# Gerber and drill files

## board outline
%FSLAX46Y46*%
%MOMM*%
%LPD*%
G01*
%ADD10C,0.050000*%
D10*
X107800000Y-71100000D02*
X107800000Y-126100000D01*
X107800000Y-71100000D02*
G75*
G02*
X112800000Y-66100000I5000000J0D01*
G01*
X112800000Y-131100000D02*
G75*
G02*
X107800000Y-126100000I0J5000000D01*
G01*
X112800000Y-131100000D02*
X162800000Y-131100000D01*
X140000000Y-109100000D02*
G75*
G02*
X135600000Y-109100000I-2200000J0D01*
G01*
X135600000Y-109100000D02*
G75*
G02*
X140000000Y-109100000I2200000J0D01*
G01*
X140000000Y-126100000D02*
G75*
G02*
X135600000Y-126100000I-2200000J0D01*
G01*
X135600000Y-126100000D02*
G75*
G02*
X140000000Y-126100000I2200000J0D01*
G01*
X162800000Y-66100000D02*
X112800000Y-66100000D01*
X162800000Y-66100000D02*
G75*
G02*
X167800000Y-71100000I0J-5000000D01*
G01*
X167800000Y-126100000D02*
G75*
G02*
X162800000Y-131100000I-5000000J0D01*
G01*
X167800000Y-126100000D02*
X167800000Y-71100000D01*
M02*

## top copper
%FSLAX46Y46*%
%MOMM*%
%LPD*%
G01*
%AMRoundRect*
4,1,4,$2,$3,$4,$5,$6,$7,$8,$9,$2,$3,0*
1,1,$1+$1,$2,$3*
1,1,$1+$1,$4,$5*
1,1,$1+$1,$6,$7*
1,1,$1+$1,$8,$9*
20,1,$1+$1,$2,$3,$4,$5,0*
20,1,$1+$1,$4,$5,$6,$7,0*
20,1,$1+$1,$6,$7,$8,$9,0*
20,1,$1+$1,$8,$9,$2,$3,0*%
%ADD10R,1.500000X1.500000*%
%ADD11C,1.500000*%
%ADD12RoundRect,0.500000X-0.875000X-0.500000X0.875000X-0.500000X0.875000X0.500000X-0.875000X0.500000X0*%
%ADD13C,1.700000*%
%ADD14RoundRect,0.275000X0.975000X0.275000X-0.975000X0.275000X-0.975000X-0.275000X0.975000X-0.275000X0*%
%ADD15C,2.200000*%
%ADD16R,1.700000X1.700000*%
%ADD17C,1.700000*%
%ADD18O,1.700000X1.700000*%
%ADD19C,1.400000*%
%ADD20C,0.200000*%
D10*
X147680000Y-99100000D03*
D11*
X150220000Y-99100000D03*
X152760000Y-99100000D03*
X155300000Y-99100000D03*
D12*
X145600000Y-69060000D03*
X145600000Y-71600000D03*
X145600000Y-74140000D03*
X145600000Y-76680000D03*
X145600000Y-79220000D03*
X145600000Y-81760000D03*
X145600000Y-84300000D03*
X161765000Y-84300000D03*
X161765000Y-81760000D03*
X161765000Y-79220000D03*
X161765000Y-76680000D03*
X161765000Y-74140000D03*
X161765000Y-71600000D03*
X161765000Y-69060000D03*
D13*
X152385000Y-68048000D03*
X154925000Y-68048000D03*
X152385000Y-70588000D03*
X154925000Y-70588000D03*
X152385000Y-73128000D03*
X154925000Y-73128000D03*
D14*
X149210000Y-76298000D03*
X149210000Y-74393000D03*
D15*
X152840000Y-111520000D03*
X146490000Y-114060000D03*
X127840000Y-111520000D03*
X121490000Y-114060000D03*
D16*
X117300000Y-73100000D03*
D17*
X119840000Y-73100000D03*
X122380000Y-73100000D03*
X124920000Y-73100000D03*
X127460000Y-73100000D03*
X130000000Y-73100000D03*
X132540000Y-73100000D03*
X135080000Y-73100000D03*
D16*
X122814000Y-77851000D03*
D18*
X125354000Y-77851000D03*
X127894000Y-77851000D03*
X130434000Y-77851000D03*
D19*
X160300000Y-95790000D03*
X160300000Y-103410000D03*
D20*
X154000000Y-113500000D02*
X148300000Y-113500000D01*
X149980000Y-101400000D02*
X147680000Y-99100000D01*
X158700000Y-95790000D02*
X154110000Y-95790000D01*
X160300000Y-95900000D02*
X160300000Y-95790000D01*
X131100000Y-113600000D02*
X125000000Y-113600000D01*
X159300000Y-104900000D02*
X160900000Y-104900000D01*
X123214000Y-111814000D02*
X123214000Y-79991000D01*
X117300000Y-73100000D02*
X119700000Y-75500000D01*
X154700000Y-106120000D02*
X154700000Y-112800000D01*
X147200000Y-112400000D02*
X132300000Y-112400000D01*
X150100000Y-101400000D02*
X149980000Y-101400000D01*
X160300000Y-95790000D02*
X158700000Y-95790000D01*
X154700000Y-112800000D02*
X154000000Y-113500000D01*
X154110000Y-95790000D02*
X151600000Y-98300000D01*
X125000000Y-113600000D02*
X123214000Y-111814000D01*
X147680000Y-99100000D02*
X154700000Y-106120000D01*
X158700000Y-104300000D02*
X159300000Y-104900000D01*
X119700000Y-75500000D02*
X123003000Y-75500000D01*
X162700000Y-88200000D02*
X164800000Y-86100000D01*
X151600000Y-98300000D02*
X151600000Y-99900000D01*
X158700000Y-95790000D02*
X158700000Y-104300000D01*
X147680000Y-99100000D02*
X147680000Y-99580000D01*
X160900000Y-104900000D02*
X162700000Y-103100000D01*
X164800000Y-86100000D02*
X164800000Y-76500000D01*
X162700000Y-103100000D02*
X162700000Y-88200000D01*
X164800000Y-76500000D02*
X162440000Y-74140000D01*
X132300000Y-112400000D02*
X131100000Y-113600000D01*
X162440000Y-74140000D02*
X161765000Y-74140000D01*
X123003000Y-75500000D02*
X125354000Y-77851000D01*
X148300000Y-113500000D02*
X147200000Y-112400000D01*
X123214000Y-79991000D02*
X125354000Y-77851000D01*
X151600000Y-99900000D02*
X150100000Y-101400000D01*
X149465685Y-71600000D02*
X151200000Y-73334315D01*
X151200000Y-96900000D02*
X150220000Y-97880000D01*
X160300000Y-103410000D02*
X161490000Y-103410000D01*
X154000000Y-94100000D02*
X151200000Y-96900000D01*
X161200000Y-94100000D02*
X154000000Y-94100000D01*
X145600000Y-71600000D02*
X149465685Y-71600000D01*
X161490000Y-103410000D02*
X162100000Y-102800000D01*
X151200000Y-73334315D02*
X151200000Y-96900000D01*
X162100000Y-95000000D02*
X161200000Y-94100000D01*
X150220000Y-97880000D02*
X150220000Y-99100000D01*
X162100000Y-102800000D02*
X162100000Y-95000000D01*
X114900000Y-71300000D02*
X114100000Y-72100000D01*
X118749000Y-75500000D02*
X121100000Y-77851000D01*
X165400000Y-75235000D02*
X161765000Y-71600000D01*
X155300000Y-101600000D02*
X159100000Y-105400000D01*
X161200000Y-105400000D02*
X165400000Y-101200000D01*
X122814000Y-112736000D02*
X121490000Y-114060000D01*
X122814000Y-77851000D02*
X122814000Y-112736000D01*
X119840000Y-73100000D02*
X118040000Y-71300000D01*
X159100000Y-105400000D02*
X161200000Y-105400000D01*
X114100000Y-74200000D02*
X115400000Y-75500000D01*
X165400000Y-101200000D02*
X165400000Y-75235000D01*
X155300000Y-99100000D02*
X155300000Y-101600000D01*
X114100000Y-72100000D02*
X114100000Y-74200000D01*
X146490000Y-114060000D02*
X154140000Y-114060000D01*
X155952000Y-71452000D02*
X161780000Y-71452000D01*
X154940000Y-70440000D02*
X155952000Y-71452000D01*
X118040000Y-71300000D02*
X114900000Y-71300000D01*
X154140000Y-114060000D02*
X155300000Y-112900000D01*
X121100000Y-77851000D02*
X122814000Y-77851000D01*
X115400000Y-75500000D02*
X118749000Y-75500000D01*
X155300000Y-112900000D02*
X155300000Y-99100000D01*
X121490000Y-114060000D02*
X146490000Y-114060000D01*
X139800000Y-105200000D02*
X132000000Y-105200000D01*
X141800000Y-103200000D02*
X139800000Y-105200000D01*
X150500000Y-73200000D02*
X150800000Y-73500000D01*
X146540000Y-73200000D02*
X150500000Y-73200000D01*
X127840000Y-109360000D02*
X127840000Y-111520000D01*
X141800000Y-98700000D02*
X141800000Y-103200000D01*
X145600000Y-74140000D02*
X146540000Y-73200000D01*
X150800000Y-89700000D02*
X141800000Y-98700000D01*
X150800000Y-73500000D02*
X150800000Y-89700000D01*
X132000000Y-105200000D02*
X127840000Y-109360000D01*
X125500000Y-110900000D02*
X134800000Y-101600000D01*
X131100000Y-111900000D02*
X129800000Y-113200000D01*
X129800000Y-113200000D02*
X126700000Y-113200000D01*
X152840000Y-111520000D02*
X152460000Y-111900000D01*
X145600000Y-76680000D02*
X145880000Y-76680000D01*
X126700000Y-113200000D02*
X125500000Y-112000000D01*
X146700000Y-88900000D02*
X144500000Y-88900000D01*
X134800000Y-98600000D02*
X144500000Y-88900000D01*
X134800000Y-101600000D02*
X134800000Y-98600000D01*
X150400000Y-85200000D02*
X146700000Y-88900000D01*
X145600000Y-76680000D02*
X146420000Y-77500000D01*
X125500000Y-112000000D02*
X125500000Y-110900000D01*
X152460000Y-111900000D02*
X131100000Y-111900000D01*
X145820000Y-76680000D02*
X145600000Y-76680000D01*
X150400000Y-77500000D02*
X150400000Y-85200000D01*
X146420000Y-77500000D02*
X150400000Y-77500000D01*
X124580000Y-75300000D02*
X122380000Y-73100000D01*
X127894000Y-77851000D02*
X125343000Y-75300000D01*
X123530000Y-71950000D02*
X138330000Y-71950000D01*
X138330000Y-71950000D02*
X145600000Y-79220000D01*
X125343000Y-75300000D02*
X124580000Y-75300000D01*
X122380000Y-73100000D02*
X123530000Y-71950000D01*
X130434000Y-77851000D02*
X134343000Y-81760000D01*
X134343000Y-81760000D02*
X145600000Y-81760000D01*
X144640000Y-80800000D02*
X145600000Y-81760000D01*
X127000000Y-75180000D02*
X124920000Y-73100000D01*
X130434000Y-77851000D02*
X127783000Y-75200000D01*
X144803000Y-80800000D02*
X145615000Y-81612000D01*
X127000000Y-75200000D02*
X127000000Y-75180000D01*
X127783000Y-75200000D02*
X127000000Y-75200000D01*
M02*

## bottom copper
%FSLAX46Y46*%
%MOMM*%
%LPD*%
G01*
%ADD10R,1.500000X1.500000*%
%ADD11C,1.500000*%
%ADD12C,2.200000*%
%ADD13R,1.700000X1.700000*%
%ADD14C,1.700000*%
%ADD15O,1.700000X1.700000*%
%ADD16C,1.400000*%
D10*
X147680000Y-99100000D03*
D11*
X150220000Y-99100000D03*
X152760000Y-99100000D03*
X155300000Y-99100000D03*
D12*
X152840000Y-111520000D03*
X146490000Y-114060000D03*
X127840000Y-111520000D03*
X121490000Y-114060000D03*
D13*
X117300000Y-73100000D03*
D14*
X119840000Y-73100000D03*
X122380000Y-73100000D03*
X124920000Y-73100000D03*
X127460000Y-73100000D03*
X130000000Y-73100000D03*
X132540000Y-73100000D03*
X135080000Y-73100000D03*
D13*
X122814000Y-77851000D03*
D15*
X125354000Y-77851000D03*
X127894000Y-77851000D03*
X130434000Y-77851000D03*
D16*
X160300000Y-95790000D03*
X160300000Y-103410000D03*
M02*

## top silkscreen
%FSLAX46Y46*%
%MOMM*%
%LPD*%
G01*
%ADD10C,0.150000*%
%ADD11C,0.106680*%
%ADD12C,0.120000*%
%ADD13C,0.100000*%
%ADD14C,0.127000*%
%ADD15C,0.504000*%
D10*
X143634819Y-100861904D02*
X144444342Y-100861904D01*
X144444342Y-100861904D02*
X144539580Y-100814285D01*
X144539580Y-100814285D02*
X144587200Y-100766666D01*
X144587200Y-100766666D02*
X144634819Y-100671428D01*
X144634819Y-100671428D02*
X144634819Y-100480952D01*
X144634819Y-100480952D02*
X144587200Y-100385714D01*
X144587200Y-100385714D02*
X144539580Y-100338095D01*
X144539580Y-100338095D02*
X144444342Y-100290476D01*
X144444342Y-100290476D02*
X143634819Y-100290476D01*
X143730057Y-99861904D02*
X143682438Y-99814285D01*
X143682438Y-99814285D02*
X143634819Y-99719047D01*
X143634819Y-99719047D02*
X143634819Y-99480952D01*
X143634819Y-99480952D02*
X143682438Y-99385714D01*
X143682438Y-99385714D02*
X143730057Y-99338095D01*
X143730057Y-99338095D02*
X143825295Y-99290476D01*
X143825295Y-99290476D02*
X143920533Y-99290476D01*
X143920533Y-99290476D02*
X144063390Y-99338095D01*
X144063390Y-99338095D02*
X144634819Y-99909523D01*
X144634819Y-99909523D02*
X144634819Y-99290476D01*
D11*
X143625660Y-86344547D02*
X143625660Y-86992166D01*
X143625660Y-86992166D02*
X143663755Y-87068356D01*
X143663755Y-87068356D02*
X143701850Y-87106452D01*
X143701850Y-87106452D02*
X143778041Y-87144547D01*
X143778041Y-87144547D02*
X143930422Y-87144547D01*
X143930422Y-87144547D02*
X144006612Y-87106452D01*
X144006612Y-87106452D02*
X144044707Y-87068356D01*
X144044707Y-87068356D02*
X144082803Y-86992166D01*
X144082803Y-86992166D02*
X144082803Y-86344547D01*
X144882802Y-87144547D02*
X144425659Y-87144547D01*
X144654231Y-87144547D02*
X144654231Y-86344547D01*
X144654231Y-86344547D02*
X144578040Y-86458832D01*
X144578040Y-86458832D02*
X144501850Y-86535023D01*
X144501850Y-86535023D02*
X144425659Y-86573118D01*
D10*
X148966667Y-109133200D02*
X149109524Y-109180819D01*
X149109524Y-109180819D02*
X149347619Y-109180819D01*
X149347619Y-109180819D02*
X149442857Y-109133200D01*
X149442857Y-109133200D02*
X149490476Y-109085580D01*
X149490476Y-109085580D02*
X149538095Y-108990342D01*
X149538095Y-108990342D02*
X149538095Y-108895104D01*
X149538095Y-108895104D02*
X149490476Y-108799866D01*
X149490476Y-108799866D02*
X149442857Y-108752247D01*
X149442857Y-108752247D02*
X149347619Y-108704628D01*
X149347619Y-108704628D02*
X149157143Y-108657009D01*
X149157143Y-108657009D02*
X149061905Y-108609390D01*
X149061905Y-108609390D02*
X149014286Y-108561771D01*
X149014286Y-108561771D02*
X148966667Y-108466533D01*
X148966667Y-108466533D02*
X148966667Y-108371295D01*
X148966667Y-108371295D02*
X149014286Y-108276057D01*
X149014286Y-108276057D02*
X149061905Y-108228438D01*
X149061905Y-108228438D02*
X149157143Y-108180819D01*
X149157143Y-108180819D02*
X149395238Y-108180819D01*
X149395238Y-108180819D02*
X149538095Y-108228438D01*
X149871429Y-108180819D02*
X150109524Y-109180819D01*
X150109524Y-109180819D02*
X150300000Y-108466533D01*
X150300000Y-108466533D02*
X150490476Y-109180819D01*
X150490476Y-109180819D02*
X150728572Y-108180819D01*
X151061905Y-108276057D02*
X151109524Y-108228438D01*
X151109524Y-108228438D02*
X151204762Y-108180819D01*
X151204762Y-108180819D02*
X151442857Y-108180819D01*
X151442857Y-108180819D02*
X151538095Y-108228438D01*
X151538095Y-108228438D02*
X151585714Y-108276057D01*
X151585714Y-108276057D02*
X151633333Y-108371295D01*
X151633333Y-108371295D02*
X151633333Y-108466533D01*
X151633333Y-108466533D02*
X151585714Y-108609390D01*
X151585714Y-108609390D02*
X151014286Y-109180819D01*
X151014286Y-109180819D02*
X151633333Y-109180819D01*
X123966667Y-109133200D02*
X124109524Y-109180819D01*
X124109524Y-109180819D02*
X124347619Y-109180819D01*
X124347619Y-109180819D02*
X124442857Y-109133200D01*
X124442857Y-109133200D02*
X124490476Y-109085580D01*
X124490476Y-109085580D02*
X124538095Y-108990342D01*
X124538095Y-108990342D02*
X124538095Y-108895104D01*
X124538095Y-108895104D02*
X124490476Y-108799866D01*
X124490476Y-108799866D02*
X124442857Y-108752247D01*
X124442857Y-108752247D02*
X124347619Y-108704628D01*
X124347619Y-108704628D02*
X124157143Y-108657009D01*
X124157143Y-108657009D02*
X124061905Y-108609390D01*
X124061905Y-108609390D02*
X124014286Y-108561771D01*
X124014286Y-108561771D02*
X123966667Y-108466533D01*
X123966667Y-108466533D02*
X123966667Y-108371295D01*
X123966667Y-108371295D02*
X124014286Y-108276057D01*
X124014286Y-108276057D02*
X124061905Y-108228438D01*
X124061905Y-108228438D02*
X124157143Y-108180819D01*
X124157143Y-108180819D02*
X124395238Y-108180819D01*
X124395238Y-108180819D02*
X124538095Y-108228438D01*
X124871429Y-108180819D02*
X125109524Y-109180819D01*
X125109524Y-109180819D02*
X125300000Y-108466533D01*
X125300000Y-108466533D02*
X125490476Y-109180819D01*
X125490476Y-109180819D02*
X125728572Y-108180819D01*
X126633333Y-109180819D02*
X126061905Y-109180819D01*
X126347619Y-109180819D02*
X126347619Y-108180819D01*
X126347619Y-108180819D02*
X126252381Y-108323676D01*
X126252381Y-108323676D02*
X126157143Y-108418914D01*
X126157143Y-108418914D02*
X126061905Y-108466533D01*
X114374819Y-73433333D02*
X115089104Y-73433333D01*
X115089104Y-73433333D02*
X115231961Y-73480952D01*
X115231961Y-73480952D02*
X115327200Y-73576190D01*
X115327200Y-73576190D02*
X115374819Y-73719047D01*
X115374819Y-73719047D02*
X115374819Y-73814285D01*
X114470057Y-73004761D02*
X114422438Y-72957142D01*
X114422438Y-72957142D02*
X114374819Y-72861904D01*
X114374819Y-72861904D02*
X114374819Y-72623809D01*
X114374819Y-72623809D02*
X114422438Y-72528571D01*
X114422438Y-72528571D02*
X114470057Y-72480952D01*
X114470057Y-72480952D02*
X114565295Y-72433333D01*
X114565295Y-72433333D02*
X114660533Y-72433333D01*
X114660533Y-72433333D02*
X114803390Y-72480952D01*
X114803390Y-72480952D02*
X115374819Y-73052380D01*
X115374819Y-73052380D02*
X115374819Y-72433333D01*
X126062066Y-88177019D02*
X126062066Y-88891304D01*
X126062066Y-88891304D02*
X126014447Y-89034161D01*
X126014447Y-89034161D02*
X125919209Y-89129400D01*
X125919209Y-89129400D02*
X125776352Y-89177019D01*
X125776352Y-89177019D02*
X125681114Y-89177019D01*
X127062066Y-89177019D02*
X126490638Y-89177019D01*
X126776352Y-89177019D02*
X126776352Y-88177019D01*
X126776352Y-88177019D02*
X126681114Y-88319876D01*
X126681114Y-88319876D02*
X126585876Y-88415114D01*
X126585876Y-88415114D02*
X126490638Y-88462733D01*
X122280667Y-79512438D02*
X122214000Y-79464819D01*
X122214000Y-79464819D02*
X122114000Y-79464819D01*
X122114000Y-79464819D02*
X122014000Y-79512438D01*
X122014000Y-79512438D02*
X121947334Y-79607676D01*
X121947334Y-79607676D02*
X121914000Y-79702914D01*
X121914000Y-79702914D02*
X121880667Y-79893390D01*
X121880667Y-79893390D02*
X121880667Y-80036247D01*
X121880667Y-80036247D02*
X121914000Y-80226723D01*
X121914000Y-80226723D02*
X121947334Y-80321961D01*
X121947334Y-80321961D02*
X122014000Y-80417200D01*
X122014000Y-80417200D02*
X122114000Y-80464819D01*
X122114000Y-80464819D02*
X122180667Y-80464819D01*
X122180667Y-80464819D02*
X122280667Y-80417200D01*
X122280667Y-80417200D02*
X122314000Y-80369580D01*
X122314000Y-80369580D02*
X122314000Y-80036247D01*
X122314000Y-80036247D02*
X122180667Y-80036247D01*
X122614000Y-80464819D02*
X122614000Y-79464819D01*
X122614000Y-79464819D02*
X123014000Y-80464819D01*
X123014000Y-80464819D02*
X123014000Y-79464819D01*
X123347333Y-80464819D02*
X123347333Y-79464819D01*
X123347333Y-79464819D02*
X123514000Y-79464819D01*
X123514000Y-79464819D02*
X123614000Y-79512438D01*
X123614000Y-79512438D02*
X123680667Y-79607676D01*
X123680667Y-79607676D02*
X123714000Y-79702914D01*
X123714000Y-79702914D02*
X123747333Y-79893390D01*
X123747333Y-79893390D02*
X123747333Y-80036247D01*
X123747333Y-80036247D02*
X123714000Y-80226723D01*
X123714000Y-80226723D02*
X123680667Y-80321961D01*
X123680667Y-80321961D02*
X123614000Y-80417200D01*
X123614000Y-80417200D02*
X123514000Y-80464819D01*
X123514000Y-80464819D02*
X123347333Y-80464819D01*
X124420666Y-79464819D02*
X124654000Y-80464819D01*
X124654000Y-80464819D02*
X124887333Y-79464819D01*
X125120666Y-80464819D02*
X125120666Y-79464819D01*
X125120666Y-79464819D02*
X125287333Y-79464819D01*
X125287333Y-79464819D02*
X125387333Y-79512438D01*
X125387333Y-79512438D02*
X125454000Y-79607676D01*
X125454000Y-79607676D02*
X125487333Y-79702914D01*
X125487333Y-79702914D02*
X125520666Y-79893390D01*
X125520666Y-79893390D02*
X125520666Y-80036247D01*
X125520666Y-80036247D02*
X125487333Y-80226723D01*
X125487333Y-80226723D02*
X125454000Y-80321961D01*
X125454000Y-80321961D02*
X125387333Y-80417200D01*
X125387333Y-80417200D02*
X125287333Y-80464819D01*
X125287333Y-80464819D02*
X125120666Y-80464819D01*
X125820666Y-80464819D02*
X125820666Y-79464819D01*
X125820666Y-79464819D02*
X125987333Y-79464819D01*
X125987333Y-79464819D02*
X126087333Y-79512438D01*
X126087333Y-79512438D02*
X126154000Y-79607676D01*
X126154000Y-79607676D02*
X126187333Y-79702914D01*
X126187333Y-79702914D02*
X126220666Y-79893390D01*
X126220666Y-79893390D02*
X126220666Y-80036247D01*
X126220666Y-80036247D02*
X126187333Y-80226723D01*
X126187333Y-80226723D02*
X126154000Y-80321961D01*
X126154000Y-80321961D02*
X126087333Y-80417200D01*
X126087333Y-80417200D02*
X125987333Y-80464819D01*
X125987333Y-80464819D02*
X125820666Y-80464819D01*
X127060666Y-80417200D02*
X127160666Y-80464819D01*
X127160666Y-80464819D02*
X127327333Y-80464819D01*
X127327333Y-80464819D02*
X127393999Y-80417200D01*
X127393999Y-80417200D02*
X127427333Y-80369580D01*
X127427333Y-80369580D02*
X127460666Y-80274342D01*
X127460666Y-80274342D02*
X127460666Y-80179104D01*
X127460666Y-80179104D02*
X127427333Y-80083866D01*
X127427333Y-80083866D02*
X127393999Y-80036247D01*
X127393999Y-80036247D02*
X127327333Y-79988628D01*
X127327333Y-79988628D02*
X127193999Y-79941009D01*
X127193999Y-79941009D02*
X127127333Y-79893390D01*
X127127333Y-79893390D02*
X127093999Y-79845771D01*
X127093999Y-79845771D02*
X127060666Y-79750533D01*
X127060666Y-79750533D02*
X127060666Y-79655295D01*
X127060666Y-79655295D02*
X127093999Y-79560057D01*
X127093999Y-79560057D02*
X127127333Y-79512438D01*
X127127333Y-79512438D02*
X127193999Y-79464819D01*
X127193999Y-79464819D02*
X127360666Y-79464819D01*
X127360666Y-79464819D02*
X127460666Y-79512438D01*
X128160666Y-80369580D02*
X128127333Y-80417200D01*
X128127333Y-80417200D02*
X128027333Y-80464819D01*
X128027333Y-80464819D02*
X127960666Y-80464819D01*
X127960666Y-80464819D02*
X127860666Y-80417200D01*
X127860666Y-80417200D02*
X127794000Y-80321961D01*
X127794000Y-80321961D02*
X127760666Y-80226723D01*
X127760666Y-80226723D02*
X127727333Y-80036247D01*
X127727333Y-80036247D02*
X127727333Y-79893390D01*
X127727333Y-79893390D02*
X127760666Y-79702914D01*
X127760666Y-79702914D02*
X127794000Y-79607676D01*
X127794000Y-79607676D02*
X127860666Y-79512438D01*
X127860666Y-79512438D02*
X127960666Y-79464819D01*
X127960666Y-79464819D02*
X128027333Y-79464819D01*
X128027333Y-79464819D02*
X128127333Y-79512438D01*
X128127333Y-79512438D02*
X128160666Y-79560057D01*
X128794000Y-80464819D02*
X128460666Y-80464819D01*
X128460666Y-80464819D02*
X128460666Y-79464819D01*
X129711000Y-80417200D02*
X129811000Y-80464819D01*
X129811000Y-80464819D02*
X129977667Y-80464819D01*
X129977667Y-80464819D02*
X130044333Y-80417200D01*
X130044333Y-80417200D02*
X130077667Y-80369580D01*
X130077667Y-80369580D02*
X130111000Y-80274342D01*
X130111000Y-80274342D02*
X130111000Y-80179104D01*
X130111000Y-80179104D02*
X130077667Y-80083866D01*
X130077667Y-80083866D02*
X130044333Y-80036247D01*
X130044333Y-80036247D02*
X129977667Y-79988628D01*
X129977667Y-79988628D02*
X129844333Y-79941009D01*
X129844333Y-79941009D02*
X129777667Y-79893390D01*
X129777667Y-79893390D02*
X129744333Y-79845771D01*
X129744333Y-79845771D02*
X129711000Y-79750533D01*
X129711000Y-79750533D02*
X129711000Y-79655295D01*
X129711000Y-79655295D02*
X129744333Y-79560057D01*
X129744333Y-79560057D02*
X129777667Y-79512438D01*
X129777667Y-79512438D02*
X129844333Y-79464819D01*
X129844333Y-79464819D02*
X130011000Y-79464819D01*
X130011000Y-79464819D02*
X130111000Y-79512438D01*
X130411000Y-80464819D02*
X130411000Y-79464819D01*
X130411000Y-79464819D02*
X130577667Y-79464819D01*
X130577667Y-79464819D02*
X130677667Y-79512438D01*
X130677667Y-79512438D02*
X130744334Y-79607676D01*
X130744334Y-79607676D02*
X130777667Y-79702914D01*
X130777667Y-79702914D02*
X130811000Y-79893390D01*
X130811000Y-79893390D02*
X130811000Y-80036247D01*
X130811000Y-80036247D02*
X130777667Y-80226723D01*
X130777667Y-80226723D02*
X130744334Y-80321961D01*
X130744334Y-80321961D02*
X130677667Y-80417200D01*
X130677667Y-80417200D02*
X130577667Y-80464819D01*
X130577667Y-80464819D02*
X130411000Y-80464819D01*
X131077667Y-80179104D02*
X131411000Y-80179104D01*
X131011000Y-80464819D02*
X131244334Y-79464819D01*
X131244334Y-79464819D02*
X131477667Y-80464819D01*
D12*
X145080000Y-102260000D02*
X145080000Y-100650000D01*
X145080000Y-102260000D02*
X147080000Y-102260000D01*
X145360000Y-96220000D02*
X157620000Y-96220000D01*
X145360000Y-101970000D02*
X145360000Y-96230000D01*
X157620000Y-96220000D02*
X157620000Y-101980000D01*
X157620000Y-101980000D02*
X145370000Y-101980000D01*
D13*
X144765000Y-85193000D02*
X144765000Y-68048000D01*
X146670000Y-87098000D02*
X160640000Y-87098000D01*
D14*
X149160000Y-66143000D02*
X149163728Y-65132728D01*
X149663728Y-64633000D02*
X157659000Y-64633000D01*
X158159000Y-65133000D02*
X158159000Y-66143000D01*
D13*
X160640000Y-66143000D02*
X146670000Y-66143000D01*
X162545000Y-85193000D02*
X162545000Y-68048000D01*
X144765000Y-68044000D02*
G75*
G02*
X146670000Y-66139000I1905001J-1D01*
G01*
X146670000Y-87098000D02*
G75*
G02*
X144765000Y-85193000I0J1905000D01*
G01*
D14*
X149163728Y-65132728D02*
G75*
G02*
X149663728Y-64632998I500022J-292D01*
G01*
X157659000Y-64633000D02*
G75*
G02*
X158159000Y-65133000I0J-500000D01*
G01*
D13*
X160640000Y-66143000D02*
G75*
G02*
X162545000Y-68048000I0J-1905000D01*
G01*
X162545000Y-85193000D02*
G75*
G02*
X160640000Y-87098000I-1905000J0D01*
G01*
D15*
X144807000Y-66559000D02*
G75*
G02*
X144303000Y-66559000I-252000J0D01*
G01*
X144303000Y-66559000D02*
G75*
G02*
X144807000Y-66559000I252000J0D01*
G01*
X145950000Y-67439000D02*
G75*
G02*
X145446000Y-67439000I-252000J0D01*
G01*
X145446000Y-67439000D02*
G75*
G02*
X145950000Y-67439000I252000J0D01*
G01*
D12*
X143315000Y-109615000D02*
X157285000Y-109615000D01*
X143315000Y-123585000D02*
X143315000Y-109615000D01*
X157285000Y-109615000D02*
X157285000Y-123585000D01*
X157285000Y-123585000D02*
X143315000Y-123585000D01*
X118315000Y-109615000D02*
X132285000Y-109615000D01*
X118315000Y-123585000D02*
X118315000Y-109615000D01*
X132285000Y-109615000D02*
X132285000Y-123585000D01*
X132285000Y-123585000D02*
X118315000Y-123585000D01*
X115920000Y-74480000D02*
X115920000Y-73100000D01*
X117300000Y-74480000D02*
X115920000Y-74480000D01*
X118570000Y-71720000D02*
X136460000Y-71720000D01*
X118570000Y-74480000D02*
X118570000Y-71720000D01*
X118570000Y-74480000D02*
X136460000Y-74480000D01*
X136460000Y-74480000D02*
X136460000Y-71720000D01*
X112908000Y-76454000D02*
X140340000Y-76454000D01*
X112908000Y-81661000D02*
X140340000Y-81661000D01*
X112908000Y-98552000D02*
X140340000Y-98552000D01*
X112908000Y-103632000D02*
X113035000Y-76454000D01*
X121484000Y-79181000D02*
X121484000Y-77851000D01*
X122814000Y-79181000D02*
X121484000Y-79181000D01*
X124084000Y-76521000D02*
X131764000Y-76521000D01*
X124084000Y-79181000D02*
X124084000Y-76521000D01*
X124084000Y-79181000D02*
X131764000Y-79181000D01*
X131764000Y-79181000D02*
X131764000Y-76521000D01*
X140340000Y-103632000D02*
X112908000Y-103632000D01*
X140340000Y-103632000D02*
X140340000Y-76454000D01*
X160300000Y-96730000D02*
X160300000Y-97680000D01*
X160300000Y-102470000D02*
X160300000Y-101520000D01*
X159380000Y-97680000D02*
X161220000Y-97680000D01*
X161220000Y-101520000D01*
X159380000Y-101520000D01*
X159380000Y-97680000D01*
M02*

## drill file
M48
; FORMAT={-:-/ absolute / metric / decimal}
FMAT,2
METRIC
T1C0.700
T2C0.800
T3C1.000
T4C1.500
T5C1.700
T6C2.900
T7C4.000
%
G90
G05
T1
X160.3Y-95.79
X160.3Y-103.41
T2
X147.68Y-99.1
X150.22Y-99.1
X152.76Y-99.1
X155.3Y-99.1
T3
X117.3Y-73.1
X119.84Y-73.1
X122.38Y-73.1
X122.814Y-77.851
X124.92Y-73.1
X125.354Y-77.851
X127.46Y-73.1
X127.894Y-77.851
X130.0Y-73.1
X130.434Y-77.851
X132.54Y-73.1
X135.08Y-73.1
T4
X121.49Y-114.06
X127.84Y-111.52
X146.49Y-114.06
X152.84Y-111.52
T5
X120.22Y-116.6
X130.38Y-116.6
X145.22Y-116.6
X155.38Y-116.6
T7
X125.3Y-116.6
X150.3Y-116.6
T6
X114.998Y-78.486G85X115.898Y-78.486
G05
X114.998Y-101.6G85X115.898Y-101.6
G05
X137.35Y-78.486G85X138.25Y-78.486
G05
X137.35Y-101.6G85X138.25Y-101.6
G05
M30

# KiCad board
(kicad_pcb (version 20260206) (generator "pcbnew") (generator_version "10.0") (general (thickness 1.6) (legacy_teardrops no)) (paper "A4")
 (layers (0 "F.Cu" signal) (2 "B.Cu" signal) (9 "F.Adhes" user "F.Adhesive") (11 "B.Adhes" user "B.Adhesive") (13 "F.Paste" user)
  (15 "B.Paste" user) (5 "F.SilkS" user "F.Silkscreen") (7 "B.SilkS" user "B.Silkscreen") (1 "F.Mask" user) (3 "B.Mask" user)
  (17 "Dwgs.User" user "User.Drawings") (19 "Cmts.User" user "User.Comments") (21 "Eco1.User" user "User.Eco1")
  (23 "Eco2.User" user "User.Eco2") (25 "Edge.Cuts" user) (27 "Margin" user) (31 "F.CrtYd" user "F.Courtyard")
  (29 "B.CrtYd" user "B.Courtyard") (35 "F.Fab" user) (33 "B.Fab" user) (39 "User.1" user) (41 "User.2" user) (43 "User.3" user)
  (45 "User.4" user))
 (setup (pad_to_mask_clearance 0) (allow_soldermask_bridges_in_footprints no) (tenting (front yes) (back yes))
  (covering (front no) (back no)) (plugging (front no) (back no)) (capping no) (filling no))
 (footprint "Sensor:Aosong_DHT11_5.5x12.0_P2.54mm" (layer "F.Cu") (at 147.68 99.1 90)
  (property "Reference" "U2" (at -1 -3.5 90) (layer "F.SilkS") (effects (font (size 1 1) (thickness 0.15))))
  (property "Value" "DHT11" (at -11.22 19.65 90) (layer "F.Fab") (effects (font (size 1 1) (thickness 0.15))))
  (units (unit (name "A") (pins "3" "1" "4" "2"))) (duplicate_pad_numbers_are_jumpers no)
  (fp_line (start -3.16 -2.6) (end -1.55 -2.6) (stroke (width 0.12) (type solid)) (layer "F.SilkS"))
  (fp_line (start -3.16 -2.6) (end -3.16 -0.6) (stroke (width 0.12) (type solid)) (layer "F.SilkS"))
  (fp_line (start 2.88 -2.32) (end 2.88 9.94) (stroke (width 0.12) (type solid)) (layer "F.SilkS"))
  (fp_line (start -2.87 -2.32) (end 2.87 -2.32) (stroke (width 0.12) (type solid)) (layer "F.SilkS"))
  (fp_line (start 2.88 9.94) (end -2.88 9.94) (stroke (width 0.12) (type solid)) (layer "F.SilkS"))
  (fp_line (start -2.88 9.94) (end -2.88 -2.31) (stroke (width 0.12) (type solid)) (layer "F.SilkS"))
  (pad "1" thru_hole rect (at 0 0 90) (size 1.5 1.5) (drill 0.8) (layers "*.Cu" "*.Mask") (remove_unused_layers no) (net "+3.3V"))
  (pad "2" thru_hole circle (at 0 2.54 90) (size 1.5 1.5) (drill 0.8) (layers "*.Cu" "*.Mask") (remove_unused_layers no) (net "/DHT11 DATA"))
  (pad "3" thru_hole circle (at 0 5.08 90) (size 1.5 1.5) (drill 0.8) (layers "*.Cu" "*.Mask") (remove_unused_layers no)
   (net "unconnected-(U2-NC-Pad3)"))
  (pad "4" thru_hole circle (at 0 7.62 90) (size 1.5 1.5) (drill 0.8) (layers "*.Cu" "*.Mask") (remove_unused_layers no) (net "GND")))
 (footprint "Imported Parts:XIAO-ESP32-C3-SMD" (layer "F.Cu") (at 144.765 87.18)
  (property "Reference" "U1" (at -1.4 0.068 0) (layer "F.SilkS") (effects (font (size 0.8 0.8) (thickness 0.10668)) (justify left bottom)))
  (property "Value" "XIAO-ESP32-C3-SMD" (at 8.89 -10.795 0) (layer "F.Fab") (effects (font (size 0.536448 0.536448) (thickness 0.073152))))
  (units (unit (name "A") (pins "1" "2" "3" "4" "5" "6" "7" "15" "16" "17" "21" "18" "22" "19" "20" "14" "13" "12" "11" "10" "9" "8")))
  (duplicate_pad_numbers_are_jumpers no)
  (fp_line (start 0 -1.987) (end 0 -19.132) (stroke (width 0.1) (type solid)) (layer "F.SilkS"))
  (fp_line (start 1.905 -0.082) (end 15.875 -0.082) (stroke (width 0.1) (type solid)) (layer "F.SilkS"))
  (fp_line (start 4.395 -21.037) (end 4.398728 -22.047272) (stroke (width 0.127) (type solid)) (layer "F.SilkS"))
  (fp_line (start 4.898728 -22.547) (end 12.894 -22.547) (stroke (width 0.127) (type solid)) (layer "F.SilkS"))
  (fp_line (start 13.394 -22.047) (end 13.394 -21.037) (stroke (width 0.127) (type solid)) (layer "F.SilkS"))
  (fp_line (start 15.875 -21.037) (end 1.905 -21.037) (stroke (width 0.1) (type solid)) (layer "F.SilkS"))
  (fp_line (start 17.78 -1.987) (end 17.78 -19.132) (stroke (width 0.1) (type solid)) (layer "F.SilkS"))
  (fp_arc (start 0 -19.136) (mid 0.557962 -20.483038) (end 1.905 -21.041) (stroke (width 0.1) (type solid)) (layer "F.SilkS"))
  (fp_arc (start 1.905 -0.082) (mid 0.557962 -0.639962) (end 0 -1.987) (stroke (width 0.1) (type solid)) (layer "F.SilkS"))
  (fp_arc (start 4.398728 -22.047272) (mid 4.545272 -22.40064) (end 4.898728 -22.547) (stroke (width 0.127) (type default))
   (layer "F.SilkS"))
  (fp_arc (start 12.894 -22.547) (mid 13.247553 -22.400553) (end 13.394 -22.047) (stroke (width 0.127) (type default)) (layer "F.SilkS"))
  (fp_arc (start 15.875 -21.037) (mid 17.222038 -20.479038) (end 17.78 -19.132) (stroke (width 0.1) (type solid)) (layer "F.SilkS"))
  (fp_arc (start 17.78 -1.987) (mid 17.222038 -0.639962) (end 15.875 -0.082) (stroke (width 0.1) (type solid)) (layer "F.SilkS"))
  (fp_circle (center -0.21 -20.621) (end -0.21 -20.875) (stroke (width 0.5) (type solid)) (fill yes) (layer "F.SilkS"))
  (fp_circle (center 0.933 -19.741) (end 0.933 -19.995) (stroke (width 0.5) (type solid)) (fill yes) (layer "F.SilkS"))
  (pad "1" smd roundrect (at 0.835 -18.12) (size 2.75 2) (layers "F.Cu" "F.Mask" "F.Paste") (roundrect_rratio 0.25)
   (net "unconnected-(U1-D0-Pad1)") (solder_mask_margin 0.0508) (thermal_bridge_angle 45))
  (pad "2" smd roundrect (at 0.835 -15.58) (size 2.75 2) (layers "F.Cu" "F.Mask" "F.Paste") (roundrect_rratio 0.25) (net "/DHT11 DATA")
   (solder_mask_margin 0.0508) (thermal_bridge_angle 45))
  (pad "3" smd roundrect (at 0.835 -13.04) (size 2.75 2) (layers "F.Cu" "F.Mask" "F.Paste") (roundrect_rratio 0.25) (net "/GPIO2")
   (solder_mask_margin 0.0508) (thermal_bridge_angle 45))
  (pad "4" smd roundrect (at 0.835 -10.5) (size 2.75 2) (layers "F.Cu" "F.Mask" "F.Paste") (roundrect_rratio 0.25) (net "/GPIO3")
   (solder_mask_margin 0.0508) (thermal_bridge_angle 45))
  (pad "5" smd roundrect (at 0.835 -7.96) (size 2.75 2) (layers "F.Cu" "F.Mask" "F.Paste") (roundrect_rratio 0.25) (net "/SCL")
   (solder_mask_margin 0.0508) (thermal_bridge_angle 45))
  (pad "6" smd roundrect (at 0.835 -5.42) (size 2.75 2) (layers "F.Cu" "F.Mask" "F.Paste") (roundrect_rratio 0.25) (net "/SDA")
   (solder_mask_margin 0.0508) (thermal_bridge_angle 45))
  (pad "7" smd roundrect (at 0.835 -2.88) (size 2.75 2) (layers "F.Cu" "F.Mask" "F.Paste") (roundrect_rratio 0.25)
   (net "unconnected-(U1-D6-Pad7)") (solder_mask_margin 0.0508) (thermal_bridge_angle 45))
  (pad "8" smd roundrect (at 17 -2.88) (size 2.75 2) (layers "F.Cu" "F.Mask" "F.Paste") (roundrect_rratio 0.25)
   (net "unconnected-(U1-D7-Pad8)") (solder_mask_margin 0.0508) (thermal_bridge_angle 45))
  (pad "9" smd roundrect (at 17 -5.42) (size 2.75 2) (layers "F.Cu" "F.Mask" "F.Paste") (roundrect_rratio 0.25)
   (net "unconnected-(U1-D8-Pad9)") (solder_mask_margin 0.0508) (thermal_bridge_angle 45))
  (pad "10" smd roundrect (at 17 -7.96) (size 2.75 2) (layers "F.Cu" "F.Mask" "F.Paste") (roundrect_rratio 0.25)
   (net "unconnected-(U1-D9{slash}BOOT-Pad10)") (solder_mask_margin 0.0508) (thermal_bridge_angle 45))
  (pad "11" smd roundrect (at 17 -10.5) (size 2.75 2) (layers "F.Cu" "F.Mask" "F.Paste") (roundrect_rratio 0.25)
   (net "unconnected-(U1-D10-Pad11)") (solder_mask_margin 0.0508) (thermal_bridge_angle 45))
  (pad "12" smd roundrect (at 17 -13.04) (size 2.75 2) (layers "F.Cu" "F.Mask" "F.Paste") (roundrect_rratio 0.25) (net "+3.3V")
   (solder_mask_margin 0.0508) (thermal_bridge_angle 45))
  (pad "13" smd roundrect (at 17 -15.58) (size 2.75 2) (layers "F.Cu" "F.Mask" "F.Paste") (roundrect_rratio 0.25) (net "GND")
   (solder_mask_margin 0.0508) (thermal_bridge_angle 45))
  (pad "14" smd roundrect (at 17 -18.12) (size 2.75 2) (layers "F.Cu" "F.Mask" "F.Paste") (roundrect_rratio 0.25) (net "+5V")
   (solder_mask_margin 0.0508) (thermal_bridge_angle 45))
  (pad "15" smd circle (at 7.62 -19.132) (size 1.7 1.7) (layers "F.Cu" "F.Mask" "F.Paste") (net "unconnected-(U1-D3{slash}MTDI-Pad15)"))
  (pad "16" smd circle (at 10.16 -19.132) (size 1.7 1.7) (layers "F.Cu" "F.Mask" "F.Paste") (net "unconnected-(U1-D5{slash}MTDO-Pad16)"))
  (pad "17" smd circle (at 7.62 -16.592) (size 1.7 1.7) (layers "F.Cu" "F.Mask" "F.Paste") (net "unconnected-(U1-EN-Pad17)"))
  (pad "18" smd circle (at 10.16 -16.592) (size 1.7 1.7) (layers "F.Cu" "F.Mask" "F.Paste") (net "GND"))
  (pad "19" smd circle (at 7.62 -14.052) (size 1.7 1.7) (layers "F.Cu" "F.Mask" "F.Paste") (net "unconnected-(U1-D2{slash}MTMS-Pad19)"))
  (pad "20" smd circle (at 10.16 -14.052) (size 1.7 1.7) (layers "F.Cu" "F.Mask" "F.Paste") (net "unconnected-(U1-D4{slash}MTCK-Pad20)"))
  (pad "21" smd roundrect (at 4.445 -10.882 180) (size 2.5 1.1) (layers "F.Cu" "F.Mask" "F.Paste") (roundrect_rratio 0.25)
   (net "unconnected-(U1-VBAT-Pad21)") (thermal_bridge_angle 45))
  (pad "22" smd roundrect (at 4.445 -12.787 180) (size 2.5 1.1) (layers "F.Cu" "F.Mask" "F.Paste") (roundrect_rratio 0.25)
   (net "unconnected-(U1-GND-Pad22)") (thermal_bridge_angle 45)))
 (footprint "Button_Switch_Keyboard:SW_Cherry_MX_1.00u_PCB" (layer "F.Cu") (at 152.84 111.52)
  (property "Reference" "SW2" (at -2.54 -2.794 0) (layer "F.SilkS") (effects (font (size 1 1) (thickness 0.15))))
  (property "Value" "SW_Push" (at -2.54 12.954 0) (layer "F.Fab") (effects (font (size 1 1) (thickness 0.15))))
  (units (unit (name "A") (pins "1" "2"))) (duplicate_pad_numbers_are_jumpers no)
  (fp_line (start -9.525 -1.905) (end 4.445 -1.905) (stroke (width 0.12) (type solid)) (layer "F.SilkS"))
  (fp_line (start -9.525 12.065) (end -9.525 -1.905) (stroke (width 0.12) (type solid)) (layer "F.SilkS"))
  (fp_line (start 4.445 -1.905) (end 4.445 12.065) (stroke (width 0.12) (type solid)) (layer "F.SilkS"))
  (fp_line (start 4.445 12.065) (end -9.525 12.065) (stroke (width 0.12) (type solid)) (layer "F.SilkS"))
  (pad "" np_thru_hole circle (at -7.62 5.08) (size 1.7 1.7) (drill 1.7) (layers "*.Cu" "*.Mask"))
  (pad "" np_thru_hole circle (at -2.54 5.08) (size 4 4) (drill 4) (layers "*.Cu" "*.Mask"))
  (pad "" np_thru_hole circle (at 2.54 5.08) (size 1.7 1.7) (drill 1.7) (layers "*.Cu" "*.Mask"))
  (pad "1" thru_hole circle (at 0 0) (size 2.2 2.2) (drill 1.5) (layers "*.Cu" "*.Mask") (remove_unused_layers no) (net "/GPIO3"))
  (pad "2" thru_hole circle (at -6.35 2.54) (size 2.2 2.2) (drill 1.5) (layers "*.Cu" "*.Mask") (remove_unused_layers no) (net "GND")))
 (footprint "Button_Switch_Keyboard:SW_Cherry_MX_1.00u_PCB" (layer "F.Cu") (at 127.84 111.52)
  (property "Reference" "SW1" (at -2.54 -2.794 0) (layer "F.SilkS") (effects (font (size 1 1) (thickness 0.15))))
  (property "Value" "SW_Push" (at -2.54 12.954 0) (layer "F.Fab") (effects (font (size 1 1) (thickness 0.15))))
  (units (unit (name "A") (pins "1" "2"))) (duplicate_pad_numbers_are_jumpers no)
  (fp_line (start -9.525 -1.905) (end 4.445 -1.905) (stroke (width 0.12) (type solid)) (layer "F.SilkS"))
  (fp_line (start -9.525 12.065) (end -9.525 -1.905) (stroke (width 0.12) (type solid)) (layer "F.SilkS"))
  (fp_line (start 4.445 -1.905) (end 4.445 12.065) (stroke (width 0.12) (type solid)) (layer "F.SilkS"))
  (fp_line (start 4.445 12.065) (end -9.525 12.065) (stroke (width 0.12) (type solid)) (layer "F.SilkS"))
  (pad "" np_thru_hole circle (at -7.62 5.08) (size 1.7 1.7) (drill 1.7) (layers "*.Cu" "*.Mask"))
  (pad "" np_thru_hole circle (at -2.54 5.08) (size 4 4) (drill 4) (layers "*.Cu" "*.Mask"))
  (pad "" np_thru_hole circle (at 2.54 5.08) (size 1.7 1.7) (drill 1.7) (layers "*.Cu" "*.Mask"))
  (pad "1" thru_hole circle (at 0 0) (size 2.2 2.2) (drill 1.5) (layers "*.Cu" "*.Mask") (remove_unused_layers no) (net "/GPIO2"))
  (pad "2" thru_hole circle (at -6.35 2.54) (size 2.2 2.2) (drill 1.5) (layers "*.Cu" "*.Mask") (remove_unused_layers no) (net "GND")))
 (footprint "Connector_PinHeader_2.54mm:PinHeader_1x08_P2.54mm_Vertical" (layer "F.Cu") (at 117.3 73.1 90)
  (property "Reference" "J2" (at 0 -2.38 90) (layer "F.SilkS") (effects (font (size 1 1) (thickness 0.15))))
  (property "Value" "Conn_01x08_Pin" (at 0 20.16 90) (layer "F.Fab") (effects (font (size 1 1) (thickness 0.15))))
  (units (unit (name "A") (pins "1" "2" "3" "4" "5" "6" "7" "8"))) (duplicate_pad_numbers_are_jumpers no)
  (fp_line (start -1.38 -1.38) (end 0 -1.38) (stroke (width 0.12) (type solid)) (layer "F.SilkS"))
  (fp_line (start -1.38 0) (end -1.38 -1.38) (stroke (width 0.12) (type solid)) (layer "F.SilkS"))
  (fp_line (start 1.38 1.27) (end 1.38 19.16) (stroke (width 0.12) (type solid)) (layer "F.SilkS"))
  (fp_line (start -1.38 1.27) (end 1.38 1.27) (stroke (width 0.12) (type solid)) (layer "F.SilkS"))
  (fp_line (start -1.38 1.27) (end -1.38 19.16) (stroke (width 0.12) (type solid)) (layer "F.SilkS"))
  (fp_line (start -1.38 19.16) (end 1.38 19.16) (stroke (width 0.12) (type solid)) (layer "F.SilkS"))
  (pad "1" thru_hole rect (at 0 0 90) (size 1.7 1.7) (drill 1) (layers "*.Cu" "*.Mask") (remove_unused_layers no) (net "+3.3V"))
  (pad "2" thru_hole circle (at 0 2.54 90) (size 1.7 1.7) (drill 1) (layers "*.Cu" "*.Mask") (remove_unused_layers no) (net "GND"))
  (pad "3" thru_hole circle (at 0 5.08 90) (size 1.7 1.7) (drill 1) (layers "*.Cu" "*.Mask") (remove_unused_layers no) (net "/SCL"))
  (pad "4" thru_hole circle (at 0 7.62 90) (size 1.7 1.7) (drill 1) (layers "*.Cu" "*.Mask") (remove_unused_layers no) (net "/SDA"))
  (pad "5" thru_hole circle (at 0 10.16 90) (size 1.7 1.7) (drill 1) (layers "*.Cu" "*.Mask") (remove_unused_layers no)
   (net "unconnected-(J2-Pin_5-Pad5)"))
  (pad "6" thru_hole circle (at 0 12.7 90) (size 1.7 1.7) (drill 1) (layers "*.Cu" "*.Mask") (remove_unused_layers no)
   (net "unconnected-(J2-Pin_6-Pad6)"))
  (pad "7" thru_hole circle (at 0 15.24 90) (size 1.7 1.7) (drill 1) (layers "*.Cu" "*.Mask") (remove_unused_layers no)
   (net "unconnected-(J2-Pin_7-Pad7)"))
  (pad "8" thru_hole circle (at 0 17.78 90) (size 1.7 1.7) (drill 1) (layers "*.Cu" "*.Mask") (remove_unused_layers no)
   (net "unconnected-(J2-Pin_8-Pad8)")))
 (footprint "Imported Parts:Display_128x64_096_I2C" (layer "F.Cu") (at 126.624 77.851)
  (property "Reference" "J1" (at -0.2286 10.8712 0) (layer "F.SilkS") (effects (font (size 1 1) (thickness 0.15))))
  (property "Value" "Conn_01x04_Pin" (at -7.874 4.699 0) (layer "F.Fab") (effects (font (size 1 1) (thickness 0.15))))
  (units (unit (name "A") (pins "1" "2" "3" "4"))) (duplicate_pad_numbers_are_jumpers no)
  (fp_line (start -13.716 -1.397) (end 13.716 -1.397) (stroke (width 0.12) (type solid)) (layer "F.SilkS"))
  (fp_line (start -13.716 3.81) (end 13.716 3.81) (stroke (width 0.12) (type solid)) (layer "F.SilkS"))
  (fp_line (start -13.716 20.701) (end 13.716 20.701) (stroke (width 0.12) (type solid)) (layer "F.SilkS"))
  (fp_line (start -13.716 25.781) (end -13.589 -1.397) (stroke (width 0.12) (type solid)) (layer "F.SilkS"))
  (fp_line (start -5.14 1.33) (end -5.14 0) (stroke (width 0.12) (type solid)) (layer "F.SilkS"))
  (fp_line (start -3.81 1.33) (end -5.14 1.33) (stroke (width 0.12) (type solid)) (layer "F.SilkS"))
  (fp_line (start -2.54 -1.33) (end 5.14 -1.33) (stroke (width 0.12) (type solid)) (layer "F.SilkS"))
  (fp_line (start -2.54 1.33) (end -2.54 -1.33) (stroke (width 0.12) (type solid)) (layer "F.SilkS"))
  (fp_line (start -2.54 1.33) (end 5.14 1.33) (stroke (width 0.12) (type solid)) (layer "F.SilkS"))
  (fp_line (start 5.14 1.33) (end 5.14 -1.33) (stroke (width 0.12) (type solid)) (layer "F.SilkS"))
  (fp_line (start 13.716 25.781) (end -13.716 25.781) (stroke (width 0.12) (type solid)) (layer "F.SilkS"))
  (fp_line (start 13.716 25.781) (end 13.716 -1.397) (stroke (width 0.12) (type solid)) (layer "F.SilkS"))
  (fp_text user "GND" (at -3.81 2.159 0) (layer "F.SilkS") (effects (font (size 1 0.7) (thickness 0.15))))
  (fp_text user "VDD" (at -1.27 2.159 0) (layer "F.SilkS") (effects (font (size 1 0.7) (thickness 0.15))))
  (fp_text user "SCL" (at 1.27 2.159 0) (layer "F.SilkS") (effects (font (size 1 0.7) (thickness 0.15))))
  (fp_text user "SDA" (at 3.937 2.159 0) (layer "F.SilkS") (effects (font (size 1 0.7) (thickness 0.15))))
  (pad "" np_thru_hole oval (at -11.176 0.635) (size 3.8 2.9) (drill oval 3.8 2.9) (layers "*.Cu" "*.Mask"))
  (pad "" np_thru_hole oval (at -11.176 23.749) (size 3.8 2.9) (drill oval 3.8 2.9) (layers "*.Cu" "*.Mask"))
  (pad "" np_thru_hole oval (at 11.176 0.635) (size 3.8 2.9) (drill oval 3.8 2.9) (layers "*.Cu" "*.Mask"))
  (pad "" np_thru_hole oval (at 11.176 23.749) (size 3.8 2.9) (drill oval 3.8 2.9) (layers "*.Cu" "*.Mask"))
  (pad "1" thru_hole rect (at -3.81 0 90) (size 1.7 1.7) (drill 1) (layers "*.Cu" "*.Mask") (remove_unused_layers no) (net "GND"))
  (pad "2" thru_hole oval (at -1.27 0 90) (size 1.7 1.7) (drill 1) (layers "*.Cu" "*.Mask") (remove_unused_layers no) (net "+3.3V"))
  (pad "3" thru_hole oval (at 1.27 0 90) (size 1.7 1.7) (drill 1) (layers "*.Cu" "*.Mask") (remove_unused_layers no) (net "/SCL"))
  (pad "4" thru_hole oval (at 3.81 0 90) (size 1.7 1.7) (drill 1) (layers "*.Cu" "*.Mask") (remove_unused_layers no) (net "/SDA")))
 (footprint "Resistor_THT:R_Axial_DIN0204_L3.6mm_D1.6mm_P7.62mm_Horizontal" (layer "F.Cu") (at 160.3 95.79 -90)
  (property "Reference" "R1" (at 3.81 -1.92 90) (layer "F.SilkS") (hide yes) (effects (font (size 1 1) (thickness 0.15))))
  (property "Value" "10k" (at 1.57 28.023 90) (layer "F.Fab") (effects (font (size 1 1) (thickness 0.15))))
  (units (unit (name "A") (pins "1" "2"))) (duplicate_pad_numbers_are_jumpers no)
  (fp_line (start 0.94 0) (end 1.89 0) (stroke (width 0.12) (type solid)) (layer "F.SilkS"))
  (fp_line (start 6.68 0) (end 5.73 0) (stroke (width 0.12) (type solid)) (layer "F.SilkS"))
  (fp_rect (start 1.89 -0.92) (end 5.73 0.92) (stroke (width 0.12) (type solid)) (fill no) (layer "F.SilkS"))
  (pad "1" thru_hole circle (at 0 0 270) (size 1.4 1.4) (drill 0.7) (layers "*.Cu" "*.Mask") (remove_unused_layers no) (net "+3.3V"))
  (pad "2" thru_hole circle (at 7.62 0 270) (size 1.4 1.4) (drill 0.7) (layers "*.Cu" "*.Mask") (remove_unused_layers no)
   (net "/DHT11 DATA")))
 (gr_line (start 107.8 71.1) (end 107.8 126.1) (stroke (width 0.05) (type default)) (layer "Edge.Cuts"))
 (gr_arc (start 107.8 71.1) (mid 109.264466 67.564466) (end 112.8 66.1) (stroke (width 0.05) (type default)) (layer "Edge.Cuts"))
 (gr_arc (start 112.8 131.1) (mid 109.264466 129.635534) (end 107.8 126.1) (stroke (width 0.05) (type default)) (layer "Edge.Cuts"))
 (gr_line (start 112.8 131.1) (end 162.8 131.1) (stroke (width 0.05) (type default)) (layer "Edge.Cuts"))
 (gr_circle (center 137.8 109.1) (end 140 109.1) (stroke (width 0.05) (type default)) (fill no) (layer "Edge.Cuts"))
 (gr_circle (center 137.8 126.1) (end 140 126.1) (stroke (width 0.05) (type default)) (fill no) (layer "Edge.Cuts"))
 (gr_line (start 162.8 66.1) (end 112.8 66.1) (stroke (width 0.05) (type default)) (layer "Edge.Cuts"))
 (gr_arc (start 162.8 66.1) (mid 166.335534 67.564466) (end 167.8 71.1) (stroke (width 0.05) (type default)) (layer "Edge.Cuts"))
 (gr_arc (start 167.8 126.1) (mid 166.335534 129.635534) (end 162.8 131.1) (stroke (width 0.05) (type default)) (layer "Edge.Cuts"))
 (gr_line (start 167.8 126.1) (end 167.8 71.1) (stroke (width 0.05) (type default)) (layer "Edge.Cuts"))
 (segment (start 154 113.5) (end 148.3 113.5) (width 0.2) (layer "F.Cu") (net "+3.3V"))
 (segment (start 149.98 101.4) (end 147.68 99.1) (width 0.2) (layer "F.Cu") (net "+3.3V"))
 (segment (start 158.7 95.79) (end 154.11 95.79) (width 0.2) (layer "F.Cu") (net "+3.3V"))
 (segment (start 160.3 95.9) (end 160.3 95.79) (width 0.2) (layer "F.Cu") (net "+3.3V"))
 (segment (start 131.1 113.6) (end 125 113.6) (width 0.2) (layer "F.Cu") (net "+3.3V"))
 (segment (start 159.3 104.9) (end 160.9 104.9) (width 0.2) (layer "F.Cu") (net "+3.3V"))
 (segment (start 123.214 111.814) (end 123.214 79.991) (width 0.2) (layer "F.Cu") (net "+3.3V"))
 (segment (start 117.3 73.1) (end 119.7 75.5) (width 0.2) (layer "F.Cu") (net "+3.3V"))
 (segment (start 154.7 106.12) (end 154.7 112.8) (width 0.2) (layer "F.Cu") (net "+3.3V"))
 (segment (start 147.2 112.4) (end 132.3 112.4) (width 0.2) (layer "F.Cu") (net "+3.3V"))
 (segment (start 150.1 101.4) (end 149.98 101.4) (width 0.2) (layer "F.Cu") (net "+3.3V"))
 (segment (start 160.3 95.79) (end 158.7 95.79) (width 0.2) (layer "F.Cu") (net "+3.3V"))
 (segment (start 154.7 112.8) (end 154 113.5) (width 0.2) (layer "F.Cu") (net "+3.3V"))
 (segment (start 154.11 95.79) (end 151.6 98.3) (width 0.2) (layer "F.Cu") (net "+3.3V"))
 (segment (start 125 113.6) (end 123.214 111.814) (width 0.2) (layer "F.Cu") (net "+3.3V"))
 (segment (start 147.68 99.1) (end 154.7 106.12) (width 0.2) (layer "F.Cu") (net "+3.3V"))
 (segment (start 158.7 104.3) (end 159.3 104.9) (width 0.2) (layer "F.Cu") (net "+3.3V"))
 (segment (start 119.7 75.5) (end 123.003 75.5) (width 0.2) (layer "F.Cu") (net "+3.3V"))
 (segment (start 162.7 88.2) (end 164.8 86.1) (width 0.2) (layer "F.Cu") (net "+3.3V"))
 (segment (start 151.6 98.3) (end 151.6 99.9) (width 0.2) (layer "F.Cu") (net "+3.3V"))
 (segment (start 158.7 95.79) (end 158.7 104.3) (width 0.2) (layer "F.Cu") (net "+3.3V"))
 (segment (start 147.68 99.1) (end 147.68 99.58) (width 0.2) (layer "F.Cu") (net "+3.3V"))
 (segment (start 160.9 104.9) (end 162.7 103.1) (width 0.2) (layer "F.Cu") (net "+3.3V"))
 (segment (start 164.8 86.1) (end 164.8 76.5) (width 0.2) (layer "F.Cu") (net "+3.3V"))
 (segment (start 162.7 103.1) (end 162.7 88.2) (width 0.2) (layer "F.Cu") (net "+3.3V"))
 (segment (start 164.8 76.5) (end 162.44 74.14) (width 0.2) (layer "F.Cu") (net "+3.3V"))
 (segment (start 132.3 112.4) (end 131.1 113.6) (width 0.2) (layer "F.Cu") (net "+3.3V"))
 (segment (start 162.44 74.14) (end 161.765 74.14) (width 0.2) (layer "F.Cu") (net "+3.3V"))
 (segment (start 123.003 75.5) (end 125.354 77.851) (width 0.2) (layer "F.Cu") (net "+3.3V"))
 (segment (start 148.3 113.5) (end 147.2 112.4) (width 0.2) (layer "F.Cu") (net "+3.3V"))
 (segment (start 123.214 79.991) (end 125.354 77.851) (width 0.2) (layer "F.Cu") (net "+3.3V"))
 (segment (start 151.6 99.9) (end 150.1 101.4) (width 0.2) (layer "F.Cu") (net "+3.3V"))
 (segment (start 149.465685 71.6) (end 151.2 73.334315) (width 0.2) (layer "F.Cu") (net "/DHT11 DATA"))
 (segment (start 151.2 96.9) (end 150.22 97.88) (width 0.2) (layer "F.Cu") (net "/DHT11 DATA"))
 (segment (start 160.3 103.41) (end 161.49 103.41) (width 0.2) (layer "F.Cu") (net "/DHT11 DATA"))
 (segment (start 154 94.1) (end 151.2 96.9) (width 0.2) (layer "F.Cu") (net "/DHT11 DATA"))
 (segment (start 161.2 94.1) (end 154 94.1) (width 0.2) (layer "F.Cu") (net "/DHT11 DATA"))
 (segment (start 145.6 71.6) (end 149.465685 71.6) (width 0.2) (layer "F.Cu") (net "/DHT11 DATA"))
 (segment (start 161.49 103.41) (end 162.1 102.8) (width 0.2) (layer "F.Cu") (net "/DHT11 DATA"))
 (segment (start 151.2 73.334315) (end 151.2 96.9) (width 0.2) (layer "F.Cu") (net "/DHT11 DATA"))
 (segment (start 162.1 95) (end 161.2 94.1) (width 0.2) (layer "F.Cu") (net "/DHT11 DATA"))
 (segment (start 150.22 97.88) (end 150.22 99.1) (width 0.2) (layer "F.Cu") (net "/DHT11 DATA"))
 (segment (start 162.1 102.8) (end 162.1 95) (width 0.2) (layer "F.Cu") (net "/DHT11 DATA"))
 (segment (start 114.9 71.3) (end 114.1 72.1) (width 0.2) (layer "F.Cu") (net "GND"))
 (segment (start 118.749 75.5) (end 121.1 77.851) (width 0.2) (layer "F.Cu") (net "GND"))
 (segment (start 165.4 75.235) (end 161.765 71.6) (width 0.2) (layer "F.Cu") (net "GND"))
 (segment (start 155.3 101.6) (end 159.1 105.4) (width 0.2) (layer "F.Cu") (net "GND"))
 (segment (start 161.2 105.4) (end 165.4 101.2) (width 0.2) (layer "F.Cu") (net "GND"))
 (segment (start 122.814 112.736) (end 121.49 114.06) (width 0.2) (layer "F.Cu") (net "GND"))
 (segment (start 122.814 77.851) (end 122.814 112.736) (width 0.2) (layer "F.Cu") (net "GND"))
 (segment (start 119.84 73.1) (end 118.04 71.3) (width 0.2) (layer "F.Cu") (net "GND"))
 (segment (start 159.1 105.4) (end 161.2 105.4) (width 0.2) (layer "F.Cu") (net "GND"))
 (segment (start 114.1 74.2) (end 115.4 75.5) (width 0.2) (layer "F.Cu") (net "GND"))
 (segment (start 165.4 101.2) (end 165.4 75.235) (width 0.2) (layer "F.Cu") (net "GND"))
 (segment (start 155.3 99.1) (end 155.3 101.6) (width 0.2) (layer "F.Cu") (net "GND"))
 (segment (start 114.1 72.1) (end 114.1 74.2) (width 0.2) (layer "F.Cu") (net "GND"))
 (segment (start 146.49 114.06) (end 154.14 114.06) (width 0.2) (layer "F.Cu") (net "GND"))
 (segment (start 155.952 71.452) (end 161.78 71.452) (width 0.2) (layer "F.Cu") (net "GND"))
 (segment (start 154.94 70.44) (end 155.952 71.452) (width 0.2) (layer "F.Cu") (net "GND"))
 (segment (start 118.04 71.3) (end 114.9 71.3) (width 0.2) (layer "F.Cu") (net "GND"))
 (segment (start 154.14 114.06) (end 155.3 112.9) (width 0.2) (layer "F.Cu") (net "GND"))
 (segment (start 121.1 77.851) (end 122.814 77.851) (width 0.2) (layer "F.Cu") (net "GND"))
 (segment (start 115.4 75.5) (end 118.749 75.5) (width 0.2) (layer "F.Cu") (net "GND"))
 (segment (start 155.3 112.9) (end 155.3 99.1) (width 0.2) (layer "F.Cu") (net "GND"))
 (segment (start 121.49 114.06) (end 146.49 114.06) (width 0.2) (layer "F.Cu") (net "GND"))
 (segment (start 139.8 105.2) (end 132 105.2) (width 0.2) (layer "F.Cu") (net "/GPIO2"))
 (segment (start 141.8 103.2) (end 139.8 105.2) (width 0.2) (layer "F.Cu") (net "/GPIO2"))
 (segment (start 150.5 73.2) (end 150.8 73.5) (width 0.2) (layer "F.Cu") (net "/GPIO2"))
 (segment (start 146.54 73.2) (end 150.5 73.2) (width 0.2) (layer "F.Cu") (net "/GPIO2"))
 (segment (start 127.84 109.36) (end 127.84 111.52) (width 0.2) (layer "F.Cu") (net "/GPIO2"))
 (segment (start 141.8 98.7) (end 141.8 103.2) (width 0.2) (layer "F.Cu") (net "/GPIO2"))
 (segment (start 145.6 74.14) (end 146.54 73.2) (width 0.2) (layer "F.Cu") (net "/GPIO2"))
 (segment (start 150.8 89.7) (end 141.8 98.7) (width 0.2) (layer "F.Cu") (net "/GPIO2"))
 (segment (start 150.8 73.5) (end 150.8 89.7) (width 0.2) (layer "F.Cu") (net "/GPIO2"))
 (segment (start 132 105.2) (end 127.84 109.36) (width 0.2) (layer "F.Cu") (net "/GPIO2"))
 (segment (start 125.5 110.9) (end 134.8 101.6) (width 0.2) (layer "F.Cu") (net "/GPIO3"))
 (segment (start 131.1 111.9) (end 129.8 113.2) (width 0.2) (layer "F.Cu") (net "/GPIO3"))
 (segment (start 129.8 113.2) (end 126.7 113.2) (width 0.2) (layer "F.Cu") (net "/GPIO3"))
 (segment (start 152.84 111.52) (end 152.46 111.9) (width 0.2) (layer "F.Cu") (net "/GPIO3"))
 (segment (start 145.6 76.68) (end 145.88 76.68) (width 0.2) (layer "F.Cu") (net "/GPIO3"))
 (segment (start 126.7 113.2) (end 125.5 112) (width 0.2) (layer "F.Cu") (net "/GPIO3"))
 (segment (start 146.7 88.9) (end 144.5 88.9) (width 0.2) (layer "F.Cu") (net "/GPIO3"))
 (segment (start 134.8 98.6) (end 144.5 88.9) (width 0.2) (layer "F.Cu") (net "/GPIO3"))
 (segment (start 134.8 101.6) (end 134.8 98.6) (width 0.2) (layer "F.Cu") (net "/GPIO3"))
 (segment (start 150.4 85.2) (end 146.7 88.9) (width 0.2) (layer "F.Cu") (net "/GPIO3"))
 (segment (start 145.6 76.68) (end 146.42 77.5) (width 0.2) (layer "F.Cu") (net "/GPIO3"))
 (segment (start 125.5 112) (end 125.5 110.9) (width 0.2) (layer "F.Cu") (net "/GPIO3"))
 (segment (start 152.46 111.9) (end 131.1 111.9) (width 0.2) (layer "F.Cu") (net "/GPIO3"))
 (segment (start 145.82 76.68) (end 145.6 76.68) (width 0.2) (layer "F.Cu") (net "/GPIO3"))
 (segment (start 150.4 77.5) (end 150.4 85.2) (width 0.2) (layer "F.Cu") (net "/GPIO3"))
 (segment (start 146.42 77.5) (end 150.4 77.5) (width 0.2) (layer "F.Cu") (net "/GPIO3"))
 (segment (start 124.58 75.3) (end 122.38 73.1) (width 0.2) (layer "F.Cu") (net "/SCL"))
 (segment (start 127.894 77.851) (end 125.343 75.3) (width 0.2) (layer "F.Cu") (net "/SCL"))
 (segment (start 123.53 71.95) (end 138.33 71.95) (width 0.2) (layer "F.Cu") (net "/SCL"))
 (segment (start 138.33 71.95) (end 145.6 79.22) (width 0.2) (layer "F.Cu") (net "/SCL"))
 (segment (start 125.343 75.3) (end 124.58 75.3) (width 0.2) (layer "F.Cu") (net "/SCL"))
 (segment (start 122.38 73.1) (end 123.53 71.95) (width 0.2) (layer "F.Cu") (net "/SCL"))
 (segment (start 130.434 77.851) (end 134.343 81.76) (width 0.2) (layer "F.Cu") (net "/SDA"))
 (segment (start 134.343 81.76) (end 145.6 81.76) (width 0.2) (layer "F.Cu") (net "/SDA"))
 (segment (start 144.64 80.8) (end 145.6 81.76) (width 0.2) (layer "F.Cu") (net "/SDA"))
 (segment (start 127 75.18) (end 124.92 73.1) (width 0.2) (layer "F.Cu") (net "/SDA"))
 (segment (start 130.434 77.851) (end 127.783 75.2) (width 0.2) (layer "F.Cu") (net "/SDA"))
 (segment (start 144.803 80.8) (end 145.615 81.612) (width 0.2) (layer "F.Cu") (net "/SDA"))
 (segment (start 127 75.2) (end 127 75.18) (width 0.2) (layer "F.Cu") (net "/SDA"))
 (segment (start 127.783 75.2) (end 127 75.2) (width 0.2) (layer "F.Cu") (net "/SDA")))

